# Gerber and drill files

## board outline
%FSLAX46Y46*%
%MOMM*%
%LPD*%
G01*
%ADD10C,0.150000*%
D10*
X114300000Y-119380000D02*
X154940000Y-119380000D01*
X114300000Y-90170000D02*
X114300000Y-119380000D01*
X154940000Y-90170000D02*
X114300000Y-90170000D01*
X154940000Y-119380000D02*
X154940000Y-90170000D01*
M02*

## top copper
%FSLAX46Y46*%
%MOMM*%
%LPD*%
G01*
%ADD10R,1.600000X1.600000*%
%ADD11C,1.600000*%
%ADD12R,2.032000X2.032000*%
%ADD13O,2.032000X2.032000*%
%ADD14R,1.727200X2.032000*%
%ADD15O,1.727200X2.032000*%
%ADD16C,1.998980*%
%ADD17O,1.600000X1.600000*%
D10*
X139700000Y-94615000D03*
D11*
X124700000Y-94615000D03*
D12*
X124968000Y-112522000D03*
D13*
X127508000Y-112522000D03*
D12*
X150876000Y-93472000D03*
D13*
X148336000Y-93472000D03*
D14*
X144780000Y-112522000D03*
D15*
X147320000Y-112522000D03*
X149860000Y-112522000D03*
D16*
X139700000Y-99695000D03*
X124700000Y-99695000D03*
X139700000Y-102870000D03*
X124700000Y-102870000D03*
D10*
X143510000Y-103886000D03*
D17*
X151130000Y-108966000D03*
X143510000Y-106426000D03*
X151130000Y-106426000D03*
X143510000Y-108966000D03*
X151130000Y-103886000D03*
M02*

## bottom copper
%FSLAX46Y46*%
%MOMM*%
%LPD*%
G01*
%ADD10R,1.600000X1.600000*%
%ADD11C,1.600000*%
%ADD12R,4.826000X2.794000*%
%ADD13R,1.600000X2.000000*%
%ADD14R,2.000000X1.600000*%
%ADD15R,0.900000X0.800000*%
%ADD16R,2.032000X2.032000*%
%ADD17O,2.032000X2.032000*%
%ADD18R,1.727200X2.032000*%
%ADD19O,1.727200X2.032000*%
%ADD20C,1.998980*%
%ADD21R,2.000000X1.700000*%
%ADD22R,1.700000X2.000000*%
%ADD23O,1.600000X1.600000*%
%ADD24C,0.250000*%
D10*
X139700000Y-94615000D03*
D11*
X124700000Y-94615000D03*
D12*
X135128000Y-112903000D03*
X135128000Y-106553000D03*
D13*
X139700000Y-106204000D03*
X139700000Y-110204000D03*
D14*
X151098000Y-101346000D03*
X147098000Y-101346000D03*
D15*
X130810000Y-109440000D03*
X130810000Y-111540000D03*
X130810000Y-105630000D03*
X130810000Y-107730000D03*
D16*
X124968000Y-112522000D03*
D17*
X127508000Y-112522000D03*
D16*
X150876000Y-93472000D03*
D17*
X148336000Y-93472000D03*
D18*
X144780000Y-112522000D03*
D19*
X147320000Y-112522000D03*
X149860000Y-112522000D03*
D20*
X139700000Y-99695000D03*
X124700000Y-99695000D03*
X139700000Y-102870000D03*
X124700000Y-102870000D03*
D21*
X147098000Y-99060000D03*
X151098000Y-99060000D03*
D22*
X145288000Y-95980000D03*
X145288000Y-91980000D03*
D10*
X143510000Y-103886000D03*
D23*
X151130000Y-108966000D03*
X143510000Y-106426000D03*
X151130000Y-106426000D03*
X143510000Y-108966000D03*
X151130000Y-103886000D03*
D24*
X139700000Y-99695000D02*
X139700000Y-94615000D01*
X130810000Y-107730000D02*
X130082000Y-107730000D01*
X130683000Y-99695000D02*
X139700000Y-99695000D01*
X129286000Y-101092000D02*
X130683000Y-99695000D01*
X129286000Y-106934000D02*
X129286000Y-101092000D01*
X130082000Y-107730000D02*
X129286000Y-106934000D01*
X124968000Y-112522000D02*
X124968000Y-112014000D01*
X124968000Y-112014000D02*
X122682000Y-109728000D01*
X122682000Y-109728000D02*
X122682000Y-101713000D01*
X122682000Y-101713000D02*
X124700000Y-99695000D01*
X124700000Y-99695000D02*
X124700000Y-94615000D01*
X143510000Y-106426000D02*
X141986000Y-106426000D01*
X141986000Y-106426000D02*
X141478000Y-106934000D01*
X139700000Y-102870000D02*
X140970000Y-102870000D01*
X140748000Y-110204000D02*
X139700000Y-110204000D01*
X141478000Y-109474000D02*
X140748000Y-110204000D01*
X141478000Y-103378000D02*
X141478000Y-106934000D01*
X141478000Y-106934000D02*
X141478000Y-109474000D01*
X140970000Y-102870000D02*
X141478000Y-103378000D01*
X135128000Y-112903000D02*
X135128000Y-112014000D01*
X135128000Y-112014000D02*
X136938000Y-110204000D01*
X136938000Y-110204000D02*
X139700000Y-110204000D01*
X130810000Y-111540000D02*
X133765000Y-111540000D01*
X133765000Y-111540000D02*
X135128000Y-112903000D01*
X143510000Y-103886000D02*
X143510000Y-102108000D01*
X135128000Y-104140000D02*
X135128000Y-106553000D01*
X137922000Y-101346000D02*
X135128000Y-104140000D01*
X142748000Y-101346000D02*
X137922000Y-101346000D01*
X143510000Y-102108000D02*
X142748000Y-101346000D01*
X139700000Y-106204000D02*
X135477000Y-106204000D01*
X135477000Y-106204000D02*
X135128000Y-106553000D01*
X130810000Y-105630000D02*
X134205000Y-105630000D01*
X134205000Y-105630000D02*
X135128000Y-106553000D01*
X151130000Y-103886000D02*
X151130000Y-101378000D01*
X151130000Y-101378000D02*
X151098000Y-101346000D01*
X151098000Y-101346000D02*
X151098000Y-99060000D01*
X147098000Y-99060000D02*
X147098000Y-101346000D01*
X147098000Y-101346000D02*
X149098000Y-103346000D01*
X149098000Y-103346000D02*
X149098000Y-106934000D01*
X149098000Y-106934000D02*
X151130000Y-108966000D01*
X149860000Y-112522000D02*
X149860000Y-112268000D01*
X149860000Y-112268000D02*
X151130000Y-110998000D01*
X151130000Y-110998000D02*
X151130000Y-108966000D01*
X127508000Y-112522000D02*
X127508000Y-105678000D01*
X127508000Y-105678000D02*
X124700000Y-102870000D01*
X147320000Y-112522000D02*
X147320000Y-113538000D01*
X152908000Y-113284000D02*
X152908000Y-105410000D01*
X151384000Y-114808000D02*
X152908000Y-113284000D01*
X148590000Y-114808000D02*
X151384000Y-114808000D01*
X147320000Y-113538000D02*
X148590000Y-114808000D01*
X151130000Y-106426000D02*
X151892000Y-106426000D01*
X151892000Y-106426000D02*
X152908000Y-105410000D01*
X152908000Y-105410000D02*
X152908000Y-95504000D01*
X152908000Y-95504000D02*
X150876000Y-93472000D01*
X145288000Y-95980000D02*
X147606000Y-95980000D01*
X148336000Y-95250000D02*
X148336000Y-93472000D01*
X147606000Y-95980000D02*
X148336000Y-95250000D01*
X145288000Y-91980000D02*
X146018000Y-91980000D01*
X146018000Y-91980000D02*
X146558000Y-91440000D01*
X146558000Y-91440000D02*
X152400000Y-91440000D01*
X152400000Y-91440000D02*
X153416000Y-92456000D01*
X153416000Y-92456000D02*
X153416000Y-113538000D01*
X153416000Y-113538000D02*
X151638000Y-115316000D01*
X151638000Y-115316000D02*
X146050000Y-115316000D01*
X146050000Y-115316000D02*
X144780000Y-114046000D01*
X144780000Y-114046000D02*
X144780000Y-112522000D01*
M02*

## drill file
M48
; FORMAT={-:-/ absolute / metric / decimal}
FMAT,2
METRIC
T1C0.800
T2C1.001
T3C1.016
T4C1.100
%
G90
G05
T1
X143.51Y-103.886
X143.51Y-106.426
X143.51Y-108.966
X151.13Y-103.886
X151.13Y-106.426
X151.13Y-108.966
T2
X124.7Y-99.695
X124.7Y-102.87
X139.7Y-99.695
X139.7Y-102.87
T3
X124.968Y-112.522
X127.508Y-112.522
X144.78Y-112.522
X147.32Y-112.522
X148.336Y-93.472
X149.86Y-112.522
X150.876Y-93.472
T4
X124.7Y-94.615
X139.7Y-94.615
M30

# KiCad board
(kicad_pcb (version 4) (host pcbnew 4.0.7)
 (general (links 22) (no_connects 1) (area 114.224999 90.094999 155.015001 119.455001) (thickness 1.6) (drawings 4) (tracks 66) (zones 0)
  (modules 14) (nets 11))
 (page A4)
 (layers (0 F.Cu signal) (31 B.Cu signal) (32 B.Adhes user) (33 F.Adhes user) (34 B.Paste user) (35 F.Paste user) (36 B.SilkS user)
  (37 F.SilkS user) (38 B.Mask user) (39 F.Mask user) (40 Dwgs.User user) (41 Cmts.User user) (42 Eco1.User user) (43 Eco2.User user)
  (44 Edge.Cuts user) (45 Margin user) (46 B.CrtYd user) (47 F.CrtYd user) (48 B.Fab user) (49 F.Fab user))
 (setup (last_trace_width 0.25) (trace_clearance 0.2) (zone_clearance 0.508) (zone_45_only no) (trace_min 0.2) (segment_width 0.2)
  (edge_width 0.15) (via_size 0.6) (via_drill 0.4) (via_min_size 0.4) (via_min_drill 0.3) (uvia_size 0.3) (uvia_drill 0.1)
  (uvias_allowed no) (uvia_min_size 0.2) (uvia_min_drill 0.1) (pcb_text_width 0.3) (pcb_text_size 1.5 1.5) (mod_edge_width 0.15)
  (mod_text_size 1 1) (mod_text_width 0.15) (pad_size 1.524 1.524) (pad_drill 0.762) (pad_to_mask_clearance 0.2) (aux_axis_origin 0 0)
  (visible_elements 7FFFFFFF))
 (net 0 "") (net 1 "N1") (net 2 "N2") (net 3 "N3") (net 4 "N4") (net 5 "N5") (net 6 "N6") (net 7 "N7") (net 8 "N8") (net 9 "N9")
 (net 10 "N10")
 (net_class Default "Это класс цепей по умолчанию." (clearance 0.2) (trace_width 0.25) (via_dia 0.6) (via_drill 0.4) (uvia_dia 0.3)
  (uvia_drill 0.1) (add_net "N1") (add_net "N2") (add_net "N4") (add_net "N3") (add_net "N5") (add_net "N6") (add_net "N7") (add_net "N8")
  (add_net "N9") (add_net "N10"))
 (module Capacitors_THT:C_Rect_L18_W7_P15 (layer F.Cu) (at 139.7 94.615 180)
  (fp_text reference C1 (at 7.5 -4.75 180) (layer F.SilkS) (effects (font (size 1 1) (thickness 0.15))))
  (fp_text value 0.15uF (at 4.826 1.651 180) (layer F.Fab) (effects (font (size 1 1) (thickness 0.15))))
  (pad 1 thru_hole rect (at 0 0 180) (size 1.6 1.6) (drill 1.1) (layers *.Cu *.Mask) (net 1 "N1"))
  (pad 2 thru_hole circle (at 15 0 180) (size 1.6 1.6) (drill 1.1) (layers *.Cu *.Mask) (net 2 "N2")))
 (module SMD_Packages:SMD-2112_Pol (layer B.Cu) (at 135.128 109.728 270)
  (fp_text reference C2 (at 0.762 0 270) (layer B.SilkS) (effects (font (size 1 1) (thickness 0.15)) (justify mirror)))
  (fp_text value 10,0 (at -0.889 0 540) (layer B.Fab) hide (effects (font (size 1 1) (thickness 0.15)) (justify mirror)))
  (pad 2 smd rect (at 3.175 0 270) (size 2.794 4.826) (layers B.Cu B.Paste B.Mask) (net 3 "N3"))
  (pad 1 smd rect (at -3.175 0 270) (size 2.794 4.826) (layers B.Cu B.Paste B.Mask) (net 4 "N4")))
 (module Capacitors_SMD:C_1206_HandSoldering (layer B.Cu) (at 139.7 108.204 270)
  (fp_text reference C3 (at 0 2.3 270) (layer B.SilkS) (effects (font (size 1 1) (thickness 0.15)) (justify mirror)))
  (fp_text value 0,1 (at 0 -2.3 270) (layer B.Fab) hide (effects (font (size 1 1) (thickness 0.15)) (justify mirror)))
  (pad 1 smd rect (at -2 0 270) (size 2 1.6) (layers B.Cu B.Paste B.Mask) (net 4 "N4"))
  (pad 2 smd rect (at 2 0 270) (size 2 1.6) (layers B.Cu B.Paste B.Mask) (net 3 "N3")))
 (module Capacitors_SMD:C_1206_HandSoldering (layer B.Cu) (at 149.098 101.346 180)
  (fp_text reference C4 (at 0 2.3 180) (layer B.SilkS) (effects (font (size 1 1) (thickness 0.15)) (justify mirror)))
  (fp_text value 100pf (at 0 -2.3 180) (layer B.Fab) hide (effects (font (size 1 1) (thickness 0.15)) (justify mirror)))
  (pad 1 smd rect (at -2 0 180) (size 2 1.6) (layers B.Cu B.Paste B.Mask) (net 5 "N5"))
  (pad 2 smd rect (at 2 0 180) (size 2 1.6) (layers B.Cu B.Paste B.Mask) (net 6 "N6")))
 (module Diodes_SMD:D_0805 (layer B.Cu) (at 130.81 110.49 270)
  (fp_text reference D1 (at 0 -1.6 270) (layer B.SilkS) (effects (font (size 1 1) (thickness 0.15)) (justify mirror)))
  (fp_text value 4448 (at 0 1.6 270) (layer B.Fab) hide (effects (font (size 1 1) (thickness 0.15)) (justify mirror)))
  (pad 1 smd rect (at -1.05 0 270) (size 0.8 0.9) (layers B.Cu B.Paste B.Mask) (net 1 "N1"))
  (pad 2 smd rect (at 1.05 0 270) (size 0.8 0.9) (layers B.Cu B.Paste B.Mask) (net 3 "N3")))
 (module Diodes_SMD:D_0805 (layer B.Cu) (at 130.81 106.68 270)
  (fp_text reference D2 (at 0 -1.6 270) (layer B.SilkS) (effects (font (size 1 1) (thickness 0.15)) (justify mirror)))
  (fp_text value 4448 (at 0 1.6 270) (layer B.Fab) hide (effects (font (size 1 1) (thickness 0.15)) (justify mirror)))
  (pad 1 smd rect (at -1.05 0 270) (size 0.8 0.9) (layers B.Cu B.Paste B.Mask) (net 4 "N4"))
  (pad 2 smd rect (at 1.05 0 270) (size 0.8 0.9) (layers B.Cu B.Paste B.Mask) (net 1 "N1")))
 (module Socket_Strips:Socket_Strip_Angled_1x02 (layer F.Cu) (at 124.968 112.522)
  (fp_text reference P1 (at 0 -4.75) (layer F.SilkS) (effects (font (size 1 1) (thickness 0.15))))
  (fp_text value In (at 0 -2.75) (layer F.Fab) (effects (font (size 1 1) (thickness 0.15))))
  (pad 1 thru_hole rect (at 0 0) (size 2.032 2.032) (drill 1.016) (layers *.Cu *.Mask) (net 2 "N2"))
  (pad 2 thru_hole oval (at 2.54 0) (size 2.032 2.032) (drill 1.016) (layers *.Cu *.Mask) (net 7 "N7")))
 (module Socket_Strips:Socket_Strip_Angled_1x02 (layer F.Cu) (at 150.876 93.472 180)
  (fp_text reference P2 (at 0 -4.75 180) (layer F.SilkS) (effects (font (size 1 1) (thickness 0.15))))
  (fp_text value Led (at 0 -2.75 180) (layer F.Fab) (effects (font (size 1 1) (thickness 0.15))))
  (pad 1 thru_hole rect (at 0 0 180) (size 2.032 2.032) (drill 1.016) (layers *.Cu *.Mask) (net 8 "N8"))
  (pad 2 thru_hole oval (at 2.54 0 180) (size 2.032 2.032) (drill 1.016) (layers *.Cu *.Mask) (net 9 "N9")))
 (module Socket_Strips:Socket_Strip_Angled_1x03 (layer F.Cu) (at 144.78 112.522)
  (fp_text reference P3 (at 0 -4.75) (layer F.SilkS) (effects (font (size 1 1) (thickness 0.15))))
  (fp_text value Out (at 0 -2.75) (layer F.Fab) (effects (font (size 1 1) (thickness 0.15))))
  (pad 1 thru_hole rect (at 0 0) (size 1.7272 2.032) (drill 1.016) (layers *.Cu *.Mask) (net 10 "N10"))
  (pad 2 thru_hole oval (at 2.54 0) (size 1.7272 2.032) (drill 1.016) (layers *.Cu *.Mask) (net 8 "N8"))
  (pad 3 thru_hole oval (at 5.08 0) (size 1.7272 2.032) (drill 1.016) (layers *.Cu *.Mask) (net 6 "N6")))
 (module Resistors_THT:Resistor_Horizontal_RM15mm (layer F.Cu) (at 139.7 99.695 180)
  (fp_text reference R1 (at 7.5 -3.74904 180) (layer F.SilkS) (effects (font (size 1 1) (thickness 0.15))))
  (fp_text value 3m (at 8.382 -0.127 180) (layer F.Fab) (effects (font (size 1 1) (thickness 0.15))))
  (pad 1 thru_hole circle (at 0 0 180) (size 1.99898 1.99898) (drill 1.00076) (layers *.Cu *.SilkS *.Mask) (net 1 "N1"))
  (pad 2 thru_hole circle (at 15 0 180) (size 1.99898 1.99898) (drill 1.00076) (layers *.Cu *.SilkS *.Mask) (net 2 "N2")))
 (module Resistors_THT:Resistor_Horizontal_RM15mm (layer F.Cu) (at 139.7 102.87 180)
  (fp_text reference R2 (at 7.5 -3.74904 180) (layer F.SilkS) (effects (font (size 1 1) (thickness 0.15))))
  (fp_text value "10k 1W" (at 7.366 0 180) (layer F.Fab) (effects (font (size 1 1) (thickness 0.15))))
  (pad 1 thru_hole circle (at 0 0 180) (size 1.99898 1.99898) (drill 1.00076) (layers *.Cu *.SilkS *.Mask) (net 3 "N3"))
  (pad 2 thru_hole circle (at 15 0 180) (size 1.99898 1.99898) (drill 1.00076) (layers *.Cu *.SilkS *.Mask) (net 7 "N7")))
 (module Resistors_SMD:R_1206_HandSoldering (layer B.Cu) (at 149.098 99.06)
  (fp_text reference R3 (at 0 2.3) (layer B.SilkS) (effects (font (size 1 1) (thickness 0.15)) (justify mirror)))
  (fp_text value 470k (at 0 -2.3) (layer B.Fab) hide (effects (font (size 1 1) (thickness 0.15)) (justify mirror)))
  (pad 1 smd rect (at -2 0) (size 2 1.7) (layers B.Cu B.Paste B.Mask) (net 6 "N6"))
  (pad 2 smd rect (at 2 0) (size 2 1.7) (layers B.Cu B.Paste B.Mask) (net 5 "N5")))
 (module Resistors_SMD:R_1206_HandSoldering (layer B.Cu) (at 145.288 93.98 90)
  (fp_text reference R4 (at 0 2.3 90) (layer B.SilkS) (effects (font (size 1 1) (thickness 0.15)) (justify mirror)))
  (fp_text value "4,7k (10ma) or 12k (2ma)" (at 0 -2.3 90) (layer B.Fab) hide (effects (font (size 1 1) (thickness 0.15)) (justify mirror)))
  (pad 1 smd rect (at -2 0 90) (size 2 1.7) (layers B.Cu B.Paste B.Mask) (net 9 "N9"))
  (pad 2 smd rect (at 2 0 90) (size 2 1.7) (layers B.Cu B.Paste B.Mask) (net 10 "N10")))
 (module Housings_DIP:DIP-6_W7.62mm (layer F.Cu) (at 143.51 103.886)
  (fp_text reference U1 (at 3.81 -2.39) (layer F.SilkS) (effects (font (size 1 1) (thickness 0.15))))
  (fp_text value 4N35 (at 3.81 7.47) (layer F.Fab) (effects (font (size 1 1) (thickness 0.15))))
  (pad 1 thru_hole rect (at 0 0) (size 1.6 1.6) (drill 0.8) (layers *.Cu *.Mask) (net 4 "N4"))
  (pad 4 thru_hole oval (at 7.62 5.08) (size 1.6 1.6) (drill 0.8) (layers *.Cu *.Mask) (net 6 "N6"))
  (pad 2 thru_hole oval (at 0 2.54) (size 1.6 1.6) (drill 0.8) (layers *.Cu *.Mask) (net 3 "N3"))
  (pad 5 thru_hole oval (at 7.62 2.54) (size 1.6 1.6) (drill 0.8) (layers *.Cu *.Mask) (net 8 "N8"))
  (pad 3 thru_hole oval (at 0 5.08) (size 1.6 1.6) (drill 0.8) (layers *.Cu *.Mask))
  (pad 6 thru_hole oval (at 7.62 0) (size 1.6 1.6) (drill 0.8) (layers *.Cu *.Mask) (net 5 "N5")))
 (gr_line (start 114.3 119.38) (end 154.94 119.38) (angle 90) (layer Edge.Cuts) (width 0.15))
 (gr_line (start 114.3 90.17) (end 114.3 119.38) (angle 90) (layer Edge.Cuts) (width 0.15))
 (gr_line (start 154.94 90.17) (end 114.3 90.17) (angle 90) (layer Edge.Cuts) (width 0.15))
 (gr_line (start 154.94 119.38) (end 154.94 90.17) (angle 90) (layer Edge.Cuts) (width 0.15))
 (segment (start 139.7 99.695) (end 139.7 94.615) (width 0.25) (layer B.Cu) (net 1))
 (segment (start 130.81 107.73) (end 130.082 107.73) (width 0.25) (layer B.Cu) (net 1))
 (segment (start 130.683 99.695) (end 139.7 99.695) (width 0.25) (layer B.Cu) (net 1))
 (segment (start 129.286 101.092) (end 130.683 99.695) (width 0.25) (layer B.Cu) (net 1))
 (segment (start 129.286 106.934) (end 129.286 101.092) (width 0.25) (layer B.Cu) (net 1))
 (segment (start 130.082 107.73) (end 129.286 106.934) (width 0.25) (layer B.Cu) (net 1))
 (segment (start 124.968 112.522) (end 124.968 112.014) (width 0.25) (layer B.Cu) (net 2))
 (segment (start 124.968 112.014) (end 122.682 109.728) (width 0.25) (layer B.Cu) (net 2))
 (segment (start 122.682 109.728) (end 122.682 101.713) (width 0.25) (layer B.Cu) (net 2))
 (segment (start 122.682 101.713) (end 124.7 99.695) (width 0.25) (layer B.Cu) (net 2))
 (segment (start 124.7 99.695) (end 124.7 94.615) (width 0.25) (layer B.Cu) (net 2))
 (segment (start 143.51 106.426) (end 141.986 106.426) (width 0.25) (layer B.Cu) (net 3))
 (segment (start 141.986 106.426) (end 141.478 106.934) (width 0.25) (layer B.Cu) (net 3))
 (segment (start 139.7 102.87) (end 140.97 102.87) (width 0.25) (layer B.Cu) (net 3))
 (segment (start 140.748 110.204) (end 139.7 110.204) (width 0.25) (layer B.Cu) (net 3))
 (segment (start 141.478 109.474) (end 140.748 110.204) (width 0.25) (layer B.Cu) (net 3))
 (segment (start 141.478 103.378) (end 141.478 106.934) (width 0.25) (layer B.Cu) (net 3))
 (segment (start 141.478 106.934) (end 141.478 109.474) (width 0.25) (layer B.Cu) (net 3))
 (segment (start 140.97 102.87) (end 141.478 103.378) (width 0.25) (layer B.Cu) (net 3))
 (segment (start 135.128 112.903) (end 135.128 112.014) (width 0.25) (layer B.Cu) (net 3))
 (segment (start 135.128 112.014) (end 136.938 110.204) (width 0.25) (layer B.Cu) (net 3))
 (segment (start 136.938 110.204) (end 139.7 110.204) (width 0.25) (layer B.Cu) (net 3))
 (segment (start 130.81 111.54) (end 133.765 111.54) (width 0.25) (layer B.Cu) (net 3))
 (segment (start 133.765 111.54) (end 135.128 112.903) (width 0.25) (layer B.Cu) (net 3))
 (segment (start 143.51 103.886) (end 143.51 102.108) (width 0.25) (layer B.Cu) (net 4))
 (segment (start 135.128 104.14) (end 135.128 106.553) (width 0.25) (layer B.Cu) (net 4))
 (segment (start 137.922 101.346) (end 135.128 104.14) (width 0.25) (layer B.Cu) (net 4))
 (segment (start 142.748 101.346) (end 137.922 101.346) (width 0.25) (layer B.Cu) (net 4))
 (segment (start 143.51 102.108) (end 142.748 101.346) (width 0.25) (layer B.Cu) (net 4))
 (segment (start 139.7 106.204) (end 135.477 106.204) (width 0.25) (layer B.Cu) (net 4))
 (segment (start 135.477 106.204) (end 135.128 106.553) (width 0.25) (layer B.Cu) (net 4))
 (segment (start 130.81 105.63) (end 134.205 105.63) (width 0.25) (layer B.Cu) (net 4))
 (segment (start 134.205 105.63) (end 135.128 106.553) (width 0.25) (layer B.Cu) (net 4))
 (segment (start 151.13 103.886) (end 151.13 101.378) (width 0.25) (layer B.Cu) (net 5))
 (segment (start 151.13 101.378) (end 151.098 101.346) (width 0.25) (layer B.Cu) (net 5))
 (segment (start 151.098 101.346) (end 151.098 99.06) (width 0.25) (layer B.Cu) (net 5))
 (segment (start 147.098 99.06) (end 147.098 101.346) (width 0.25) (layer B.Cu) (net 6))
 (segment (start 147.098 101.346) (end 149.098 103.346) (width 0.25) (layer B.Cu) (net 6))
 (segment (start 149.098 103.346) (end 149.098 106.934) (width 0.25) (layer B.Cu) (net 6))
 (segment (start 149.098 106.934) (end 151.13 108.966) (width 0.25) (layer B.Cu) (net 6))
 (segment (start 149.86 112.522) (end 149.86 112.268) (width 0.25) (layer B.Cu) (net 6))
 (segment (start 149.86 112.268) (end 151.13 110.998) (width 0.25) (layer B.Cu) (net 6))
 (segment (start 151.13 110.998) (end 151.13 108.966) (width 0.25) (layer B.Cu) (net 6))
 (segment (start 127.508 112.522) (end 127.508 105.678) (width 0.25) (layer B.Cu) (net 7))
 (segment (start 127.508 105.678) (end 124.7 102.87) (width 0.25) (layer B.Cu) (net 7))
 (segment (start 147.32 112.522) (end 147.32 113.538) (width 0.25) (layer B.Cu) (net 8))
 (segment (start 152.908 113.284) (end 152.908 105.41) (width 0.25) (layer B.Cu) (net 8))
 (segment (start 151.384 114.808) (end 152.908 113.284) (width 0.25) (layer B.Cu) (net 8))
 (segment (start 148.59 114.808) (end 151.384 114.808) (width 0.25) (layer B.Cu) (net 8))
 (segment (start 147.32 113.538) (end 148.59 114.808) (width 0.25) (layer B.Cu) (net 8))
 (segment (start 151.13 106.426) (end 151.892 106.426) (width 0.25) (layer B.Cu) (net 8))
 (segment (start 151.892 106.426) (end 152.908 105.41) (width 0.25) (layer B.Cu) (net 8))
 (segment (start 152.908 105.41) (end 152.908 95.504) (width 0.25) (layer B.Cu) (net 8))
 (segment (start 152.908 95.504) (end 150.876 93.472) (width 0.25) (layer B.Cu) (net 8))
 (segment (start 145.288 95.98) (end 147.606 95.98) (width 0.25) (layer B.Cu) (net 9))
 (segment (start 148.336 95.25) (end 148.336 93.472) (width 0.25) (layer B.Cu) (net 9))
 (segment (start 147.606 95.98) (end 148.336 95.25) (width 0.25) (layer B.Cu) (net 9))
 (segment (start 145.288 91.98) (end 146.018 91.98) (width 0.25) (layer B.Cu) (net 10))
 (segment (start 146.018 91.98) (end 146.558 91.44) (width 0.25) (layer B.Cu) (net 10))
 (segment (start 146.558 91.44) (end 152.4 91.44) (width 0.25) (layer B.Cu) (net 10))
 (segment (start 152.4 91.44) (end 153.416 92.456) (width 0.25) (layer B.Cu) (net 10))
 (segment (start 153.416 92.456) (end 153.416 113.538) (width 0.25) (layer B.Cu) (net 10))
 (segment (start 153.416 113.538) (end 151.638 115.316) (width 0.25) (layer B.Cu) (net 10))
 (segment (start 151.638 115.316) (end 146.05 115.316) (width 0.25) (layer B.Cu) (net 10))
 (segment (start 146.05 115.316) (end 144.78 114.046) (width 0.25) (layer B.Cu) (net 10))
 (segment (start 144.78 114.046) (end 144.78 112.522) (width 0.25) (layer B.Cu) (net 10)))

